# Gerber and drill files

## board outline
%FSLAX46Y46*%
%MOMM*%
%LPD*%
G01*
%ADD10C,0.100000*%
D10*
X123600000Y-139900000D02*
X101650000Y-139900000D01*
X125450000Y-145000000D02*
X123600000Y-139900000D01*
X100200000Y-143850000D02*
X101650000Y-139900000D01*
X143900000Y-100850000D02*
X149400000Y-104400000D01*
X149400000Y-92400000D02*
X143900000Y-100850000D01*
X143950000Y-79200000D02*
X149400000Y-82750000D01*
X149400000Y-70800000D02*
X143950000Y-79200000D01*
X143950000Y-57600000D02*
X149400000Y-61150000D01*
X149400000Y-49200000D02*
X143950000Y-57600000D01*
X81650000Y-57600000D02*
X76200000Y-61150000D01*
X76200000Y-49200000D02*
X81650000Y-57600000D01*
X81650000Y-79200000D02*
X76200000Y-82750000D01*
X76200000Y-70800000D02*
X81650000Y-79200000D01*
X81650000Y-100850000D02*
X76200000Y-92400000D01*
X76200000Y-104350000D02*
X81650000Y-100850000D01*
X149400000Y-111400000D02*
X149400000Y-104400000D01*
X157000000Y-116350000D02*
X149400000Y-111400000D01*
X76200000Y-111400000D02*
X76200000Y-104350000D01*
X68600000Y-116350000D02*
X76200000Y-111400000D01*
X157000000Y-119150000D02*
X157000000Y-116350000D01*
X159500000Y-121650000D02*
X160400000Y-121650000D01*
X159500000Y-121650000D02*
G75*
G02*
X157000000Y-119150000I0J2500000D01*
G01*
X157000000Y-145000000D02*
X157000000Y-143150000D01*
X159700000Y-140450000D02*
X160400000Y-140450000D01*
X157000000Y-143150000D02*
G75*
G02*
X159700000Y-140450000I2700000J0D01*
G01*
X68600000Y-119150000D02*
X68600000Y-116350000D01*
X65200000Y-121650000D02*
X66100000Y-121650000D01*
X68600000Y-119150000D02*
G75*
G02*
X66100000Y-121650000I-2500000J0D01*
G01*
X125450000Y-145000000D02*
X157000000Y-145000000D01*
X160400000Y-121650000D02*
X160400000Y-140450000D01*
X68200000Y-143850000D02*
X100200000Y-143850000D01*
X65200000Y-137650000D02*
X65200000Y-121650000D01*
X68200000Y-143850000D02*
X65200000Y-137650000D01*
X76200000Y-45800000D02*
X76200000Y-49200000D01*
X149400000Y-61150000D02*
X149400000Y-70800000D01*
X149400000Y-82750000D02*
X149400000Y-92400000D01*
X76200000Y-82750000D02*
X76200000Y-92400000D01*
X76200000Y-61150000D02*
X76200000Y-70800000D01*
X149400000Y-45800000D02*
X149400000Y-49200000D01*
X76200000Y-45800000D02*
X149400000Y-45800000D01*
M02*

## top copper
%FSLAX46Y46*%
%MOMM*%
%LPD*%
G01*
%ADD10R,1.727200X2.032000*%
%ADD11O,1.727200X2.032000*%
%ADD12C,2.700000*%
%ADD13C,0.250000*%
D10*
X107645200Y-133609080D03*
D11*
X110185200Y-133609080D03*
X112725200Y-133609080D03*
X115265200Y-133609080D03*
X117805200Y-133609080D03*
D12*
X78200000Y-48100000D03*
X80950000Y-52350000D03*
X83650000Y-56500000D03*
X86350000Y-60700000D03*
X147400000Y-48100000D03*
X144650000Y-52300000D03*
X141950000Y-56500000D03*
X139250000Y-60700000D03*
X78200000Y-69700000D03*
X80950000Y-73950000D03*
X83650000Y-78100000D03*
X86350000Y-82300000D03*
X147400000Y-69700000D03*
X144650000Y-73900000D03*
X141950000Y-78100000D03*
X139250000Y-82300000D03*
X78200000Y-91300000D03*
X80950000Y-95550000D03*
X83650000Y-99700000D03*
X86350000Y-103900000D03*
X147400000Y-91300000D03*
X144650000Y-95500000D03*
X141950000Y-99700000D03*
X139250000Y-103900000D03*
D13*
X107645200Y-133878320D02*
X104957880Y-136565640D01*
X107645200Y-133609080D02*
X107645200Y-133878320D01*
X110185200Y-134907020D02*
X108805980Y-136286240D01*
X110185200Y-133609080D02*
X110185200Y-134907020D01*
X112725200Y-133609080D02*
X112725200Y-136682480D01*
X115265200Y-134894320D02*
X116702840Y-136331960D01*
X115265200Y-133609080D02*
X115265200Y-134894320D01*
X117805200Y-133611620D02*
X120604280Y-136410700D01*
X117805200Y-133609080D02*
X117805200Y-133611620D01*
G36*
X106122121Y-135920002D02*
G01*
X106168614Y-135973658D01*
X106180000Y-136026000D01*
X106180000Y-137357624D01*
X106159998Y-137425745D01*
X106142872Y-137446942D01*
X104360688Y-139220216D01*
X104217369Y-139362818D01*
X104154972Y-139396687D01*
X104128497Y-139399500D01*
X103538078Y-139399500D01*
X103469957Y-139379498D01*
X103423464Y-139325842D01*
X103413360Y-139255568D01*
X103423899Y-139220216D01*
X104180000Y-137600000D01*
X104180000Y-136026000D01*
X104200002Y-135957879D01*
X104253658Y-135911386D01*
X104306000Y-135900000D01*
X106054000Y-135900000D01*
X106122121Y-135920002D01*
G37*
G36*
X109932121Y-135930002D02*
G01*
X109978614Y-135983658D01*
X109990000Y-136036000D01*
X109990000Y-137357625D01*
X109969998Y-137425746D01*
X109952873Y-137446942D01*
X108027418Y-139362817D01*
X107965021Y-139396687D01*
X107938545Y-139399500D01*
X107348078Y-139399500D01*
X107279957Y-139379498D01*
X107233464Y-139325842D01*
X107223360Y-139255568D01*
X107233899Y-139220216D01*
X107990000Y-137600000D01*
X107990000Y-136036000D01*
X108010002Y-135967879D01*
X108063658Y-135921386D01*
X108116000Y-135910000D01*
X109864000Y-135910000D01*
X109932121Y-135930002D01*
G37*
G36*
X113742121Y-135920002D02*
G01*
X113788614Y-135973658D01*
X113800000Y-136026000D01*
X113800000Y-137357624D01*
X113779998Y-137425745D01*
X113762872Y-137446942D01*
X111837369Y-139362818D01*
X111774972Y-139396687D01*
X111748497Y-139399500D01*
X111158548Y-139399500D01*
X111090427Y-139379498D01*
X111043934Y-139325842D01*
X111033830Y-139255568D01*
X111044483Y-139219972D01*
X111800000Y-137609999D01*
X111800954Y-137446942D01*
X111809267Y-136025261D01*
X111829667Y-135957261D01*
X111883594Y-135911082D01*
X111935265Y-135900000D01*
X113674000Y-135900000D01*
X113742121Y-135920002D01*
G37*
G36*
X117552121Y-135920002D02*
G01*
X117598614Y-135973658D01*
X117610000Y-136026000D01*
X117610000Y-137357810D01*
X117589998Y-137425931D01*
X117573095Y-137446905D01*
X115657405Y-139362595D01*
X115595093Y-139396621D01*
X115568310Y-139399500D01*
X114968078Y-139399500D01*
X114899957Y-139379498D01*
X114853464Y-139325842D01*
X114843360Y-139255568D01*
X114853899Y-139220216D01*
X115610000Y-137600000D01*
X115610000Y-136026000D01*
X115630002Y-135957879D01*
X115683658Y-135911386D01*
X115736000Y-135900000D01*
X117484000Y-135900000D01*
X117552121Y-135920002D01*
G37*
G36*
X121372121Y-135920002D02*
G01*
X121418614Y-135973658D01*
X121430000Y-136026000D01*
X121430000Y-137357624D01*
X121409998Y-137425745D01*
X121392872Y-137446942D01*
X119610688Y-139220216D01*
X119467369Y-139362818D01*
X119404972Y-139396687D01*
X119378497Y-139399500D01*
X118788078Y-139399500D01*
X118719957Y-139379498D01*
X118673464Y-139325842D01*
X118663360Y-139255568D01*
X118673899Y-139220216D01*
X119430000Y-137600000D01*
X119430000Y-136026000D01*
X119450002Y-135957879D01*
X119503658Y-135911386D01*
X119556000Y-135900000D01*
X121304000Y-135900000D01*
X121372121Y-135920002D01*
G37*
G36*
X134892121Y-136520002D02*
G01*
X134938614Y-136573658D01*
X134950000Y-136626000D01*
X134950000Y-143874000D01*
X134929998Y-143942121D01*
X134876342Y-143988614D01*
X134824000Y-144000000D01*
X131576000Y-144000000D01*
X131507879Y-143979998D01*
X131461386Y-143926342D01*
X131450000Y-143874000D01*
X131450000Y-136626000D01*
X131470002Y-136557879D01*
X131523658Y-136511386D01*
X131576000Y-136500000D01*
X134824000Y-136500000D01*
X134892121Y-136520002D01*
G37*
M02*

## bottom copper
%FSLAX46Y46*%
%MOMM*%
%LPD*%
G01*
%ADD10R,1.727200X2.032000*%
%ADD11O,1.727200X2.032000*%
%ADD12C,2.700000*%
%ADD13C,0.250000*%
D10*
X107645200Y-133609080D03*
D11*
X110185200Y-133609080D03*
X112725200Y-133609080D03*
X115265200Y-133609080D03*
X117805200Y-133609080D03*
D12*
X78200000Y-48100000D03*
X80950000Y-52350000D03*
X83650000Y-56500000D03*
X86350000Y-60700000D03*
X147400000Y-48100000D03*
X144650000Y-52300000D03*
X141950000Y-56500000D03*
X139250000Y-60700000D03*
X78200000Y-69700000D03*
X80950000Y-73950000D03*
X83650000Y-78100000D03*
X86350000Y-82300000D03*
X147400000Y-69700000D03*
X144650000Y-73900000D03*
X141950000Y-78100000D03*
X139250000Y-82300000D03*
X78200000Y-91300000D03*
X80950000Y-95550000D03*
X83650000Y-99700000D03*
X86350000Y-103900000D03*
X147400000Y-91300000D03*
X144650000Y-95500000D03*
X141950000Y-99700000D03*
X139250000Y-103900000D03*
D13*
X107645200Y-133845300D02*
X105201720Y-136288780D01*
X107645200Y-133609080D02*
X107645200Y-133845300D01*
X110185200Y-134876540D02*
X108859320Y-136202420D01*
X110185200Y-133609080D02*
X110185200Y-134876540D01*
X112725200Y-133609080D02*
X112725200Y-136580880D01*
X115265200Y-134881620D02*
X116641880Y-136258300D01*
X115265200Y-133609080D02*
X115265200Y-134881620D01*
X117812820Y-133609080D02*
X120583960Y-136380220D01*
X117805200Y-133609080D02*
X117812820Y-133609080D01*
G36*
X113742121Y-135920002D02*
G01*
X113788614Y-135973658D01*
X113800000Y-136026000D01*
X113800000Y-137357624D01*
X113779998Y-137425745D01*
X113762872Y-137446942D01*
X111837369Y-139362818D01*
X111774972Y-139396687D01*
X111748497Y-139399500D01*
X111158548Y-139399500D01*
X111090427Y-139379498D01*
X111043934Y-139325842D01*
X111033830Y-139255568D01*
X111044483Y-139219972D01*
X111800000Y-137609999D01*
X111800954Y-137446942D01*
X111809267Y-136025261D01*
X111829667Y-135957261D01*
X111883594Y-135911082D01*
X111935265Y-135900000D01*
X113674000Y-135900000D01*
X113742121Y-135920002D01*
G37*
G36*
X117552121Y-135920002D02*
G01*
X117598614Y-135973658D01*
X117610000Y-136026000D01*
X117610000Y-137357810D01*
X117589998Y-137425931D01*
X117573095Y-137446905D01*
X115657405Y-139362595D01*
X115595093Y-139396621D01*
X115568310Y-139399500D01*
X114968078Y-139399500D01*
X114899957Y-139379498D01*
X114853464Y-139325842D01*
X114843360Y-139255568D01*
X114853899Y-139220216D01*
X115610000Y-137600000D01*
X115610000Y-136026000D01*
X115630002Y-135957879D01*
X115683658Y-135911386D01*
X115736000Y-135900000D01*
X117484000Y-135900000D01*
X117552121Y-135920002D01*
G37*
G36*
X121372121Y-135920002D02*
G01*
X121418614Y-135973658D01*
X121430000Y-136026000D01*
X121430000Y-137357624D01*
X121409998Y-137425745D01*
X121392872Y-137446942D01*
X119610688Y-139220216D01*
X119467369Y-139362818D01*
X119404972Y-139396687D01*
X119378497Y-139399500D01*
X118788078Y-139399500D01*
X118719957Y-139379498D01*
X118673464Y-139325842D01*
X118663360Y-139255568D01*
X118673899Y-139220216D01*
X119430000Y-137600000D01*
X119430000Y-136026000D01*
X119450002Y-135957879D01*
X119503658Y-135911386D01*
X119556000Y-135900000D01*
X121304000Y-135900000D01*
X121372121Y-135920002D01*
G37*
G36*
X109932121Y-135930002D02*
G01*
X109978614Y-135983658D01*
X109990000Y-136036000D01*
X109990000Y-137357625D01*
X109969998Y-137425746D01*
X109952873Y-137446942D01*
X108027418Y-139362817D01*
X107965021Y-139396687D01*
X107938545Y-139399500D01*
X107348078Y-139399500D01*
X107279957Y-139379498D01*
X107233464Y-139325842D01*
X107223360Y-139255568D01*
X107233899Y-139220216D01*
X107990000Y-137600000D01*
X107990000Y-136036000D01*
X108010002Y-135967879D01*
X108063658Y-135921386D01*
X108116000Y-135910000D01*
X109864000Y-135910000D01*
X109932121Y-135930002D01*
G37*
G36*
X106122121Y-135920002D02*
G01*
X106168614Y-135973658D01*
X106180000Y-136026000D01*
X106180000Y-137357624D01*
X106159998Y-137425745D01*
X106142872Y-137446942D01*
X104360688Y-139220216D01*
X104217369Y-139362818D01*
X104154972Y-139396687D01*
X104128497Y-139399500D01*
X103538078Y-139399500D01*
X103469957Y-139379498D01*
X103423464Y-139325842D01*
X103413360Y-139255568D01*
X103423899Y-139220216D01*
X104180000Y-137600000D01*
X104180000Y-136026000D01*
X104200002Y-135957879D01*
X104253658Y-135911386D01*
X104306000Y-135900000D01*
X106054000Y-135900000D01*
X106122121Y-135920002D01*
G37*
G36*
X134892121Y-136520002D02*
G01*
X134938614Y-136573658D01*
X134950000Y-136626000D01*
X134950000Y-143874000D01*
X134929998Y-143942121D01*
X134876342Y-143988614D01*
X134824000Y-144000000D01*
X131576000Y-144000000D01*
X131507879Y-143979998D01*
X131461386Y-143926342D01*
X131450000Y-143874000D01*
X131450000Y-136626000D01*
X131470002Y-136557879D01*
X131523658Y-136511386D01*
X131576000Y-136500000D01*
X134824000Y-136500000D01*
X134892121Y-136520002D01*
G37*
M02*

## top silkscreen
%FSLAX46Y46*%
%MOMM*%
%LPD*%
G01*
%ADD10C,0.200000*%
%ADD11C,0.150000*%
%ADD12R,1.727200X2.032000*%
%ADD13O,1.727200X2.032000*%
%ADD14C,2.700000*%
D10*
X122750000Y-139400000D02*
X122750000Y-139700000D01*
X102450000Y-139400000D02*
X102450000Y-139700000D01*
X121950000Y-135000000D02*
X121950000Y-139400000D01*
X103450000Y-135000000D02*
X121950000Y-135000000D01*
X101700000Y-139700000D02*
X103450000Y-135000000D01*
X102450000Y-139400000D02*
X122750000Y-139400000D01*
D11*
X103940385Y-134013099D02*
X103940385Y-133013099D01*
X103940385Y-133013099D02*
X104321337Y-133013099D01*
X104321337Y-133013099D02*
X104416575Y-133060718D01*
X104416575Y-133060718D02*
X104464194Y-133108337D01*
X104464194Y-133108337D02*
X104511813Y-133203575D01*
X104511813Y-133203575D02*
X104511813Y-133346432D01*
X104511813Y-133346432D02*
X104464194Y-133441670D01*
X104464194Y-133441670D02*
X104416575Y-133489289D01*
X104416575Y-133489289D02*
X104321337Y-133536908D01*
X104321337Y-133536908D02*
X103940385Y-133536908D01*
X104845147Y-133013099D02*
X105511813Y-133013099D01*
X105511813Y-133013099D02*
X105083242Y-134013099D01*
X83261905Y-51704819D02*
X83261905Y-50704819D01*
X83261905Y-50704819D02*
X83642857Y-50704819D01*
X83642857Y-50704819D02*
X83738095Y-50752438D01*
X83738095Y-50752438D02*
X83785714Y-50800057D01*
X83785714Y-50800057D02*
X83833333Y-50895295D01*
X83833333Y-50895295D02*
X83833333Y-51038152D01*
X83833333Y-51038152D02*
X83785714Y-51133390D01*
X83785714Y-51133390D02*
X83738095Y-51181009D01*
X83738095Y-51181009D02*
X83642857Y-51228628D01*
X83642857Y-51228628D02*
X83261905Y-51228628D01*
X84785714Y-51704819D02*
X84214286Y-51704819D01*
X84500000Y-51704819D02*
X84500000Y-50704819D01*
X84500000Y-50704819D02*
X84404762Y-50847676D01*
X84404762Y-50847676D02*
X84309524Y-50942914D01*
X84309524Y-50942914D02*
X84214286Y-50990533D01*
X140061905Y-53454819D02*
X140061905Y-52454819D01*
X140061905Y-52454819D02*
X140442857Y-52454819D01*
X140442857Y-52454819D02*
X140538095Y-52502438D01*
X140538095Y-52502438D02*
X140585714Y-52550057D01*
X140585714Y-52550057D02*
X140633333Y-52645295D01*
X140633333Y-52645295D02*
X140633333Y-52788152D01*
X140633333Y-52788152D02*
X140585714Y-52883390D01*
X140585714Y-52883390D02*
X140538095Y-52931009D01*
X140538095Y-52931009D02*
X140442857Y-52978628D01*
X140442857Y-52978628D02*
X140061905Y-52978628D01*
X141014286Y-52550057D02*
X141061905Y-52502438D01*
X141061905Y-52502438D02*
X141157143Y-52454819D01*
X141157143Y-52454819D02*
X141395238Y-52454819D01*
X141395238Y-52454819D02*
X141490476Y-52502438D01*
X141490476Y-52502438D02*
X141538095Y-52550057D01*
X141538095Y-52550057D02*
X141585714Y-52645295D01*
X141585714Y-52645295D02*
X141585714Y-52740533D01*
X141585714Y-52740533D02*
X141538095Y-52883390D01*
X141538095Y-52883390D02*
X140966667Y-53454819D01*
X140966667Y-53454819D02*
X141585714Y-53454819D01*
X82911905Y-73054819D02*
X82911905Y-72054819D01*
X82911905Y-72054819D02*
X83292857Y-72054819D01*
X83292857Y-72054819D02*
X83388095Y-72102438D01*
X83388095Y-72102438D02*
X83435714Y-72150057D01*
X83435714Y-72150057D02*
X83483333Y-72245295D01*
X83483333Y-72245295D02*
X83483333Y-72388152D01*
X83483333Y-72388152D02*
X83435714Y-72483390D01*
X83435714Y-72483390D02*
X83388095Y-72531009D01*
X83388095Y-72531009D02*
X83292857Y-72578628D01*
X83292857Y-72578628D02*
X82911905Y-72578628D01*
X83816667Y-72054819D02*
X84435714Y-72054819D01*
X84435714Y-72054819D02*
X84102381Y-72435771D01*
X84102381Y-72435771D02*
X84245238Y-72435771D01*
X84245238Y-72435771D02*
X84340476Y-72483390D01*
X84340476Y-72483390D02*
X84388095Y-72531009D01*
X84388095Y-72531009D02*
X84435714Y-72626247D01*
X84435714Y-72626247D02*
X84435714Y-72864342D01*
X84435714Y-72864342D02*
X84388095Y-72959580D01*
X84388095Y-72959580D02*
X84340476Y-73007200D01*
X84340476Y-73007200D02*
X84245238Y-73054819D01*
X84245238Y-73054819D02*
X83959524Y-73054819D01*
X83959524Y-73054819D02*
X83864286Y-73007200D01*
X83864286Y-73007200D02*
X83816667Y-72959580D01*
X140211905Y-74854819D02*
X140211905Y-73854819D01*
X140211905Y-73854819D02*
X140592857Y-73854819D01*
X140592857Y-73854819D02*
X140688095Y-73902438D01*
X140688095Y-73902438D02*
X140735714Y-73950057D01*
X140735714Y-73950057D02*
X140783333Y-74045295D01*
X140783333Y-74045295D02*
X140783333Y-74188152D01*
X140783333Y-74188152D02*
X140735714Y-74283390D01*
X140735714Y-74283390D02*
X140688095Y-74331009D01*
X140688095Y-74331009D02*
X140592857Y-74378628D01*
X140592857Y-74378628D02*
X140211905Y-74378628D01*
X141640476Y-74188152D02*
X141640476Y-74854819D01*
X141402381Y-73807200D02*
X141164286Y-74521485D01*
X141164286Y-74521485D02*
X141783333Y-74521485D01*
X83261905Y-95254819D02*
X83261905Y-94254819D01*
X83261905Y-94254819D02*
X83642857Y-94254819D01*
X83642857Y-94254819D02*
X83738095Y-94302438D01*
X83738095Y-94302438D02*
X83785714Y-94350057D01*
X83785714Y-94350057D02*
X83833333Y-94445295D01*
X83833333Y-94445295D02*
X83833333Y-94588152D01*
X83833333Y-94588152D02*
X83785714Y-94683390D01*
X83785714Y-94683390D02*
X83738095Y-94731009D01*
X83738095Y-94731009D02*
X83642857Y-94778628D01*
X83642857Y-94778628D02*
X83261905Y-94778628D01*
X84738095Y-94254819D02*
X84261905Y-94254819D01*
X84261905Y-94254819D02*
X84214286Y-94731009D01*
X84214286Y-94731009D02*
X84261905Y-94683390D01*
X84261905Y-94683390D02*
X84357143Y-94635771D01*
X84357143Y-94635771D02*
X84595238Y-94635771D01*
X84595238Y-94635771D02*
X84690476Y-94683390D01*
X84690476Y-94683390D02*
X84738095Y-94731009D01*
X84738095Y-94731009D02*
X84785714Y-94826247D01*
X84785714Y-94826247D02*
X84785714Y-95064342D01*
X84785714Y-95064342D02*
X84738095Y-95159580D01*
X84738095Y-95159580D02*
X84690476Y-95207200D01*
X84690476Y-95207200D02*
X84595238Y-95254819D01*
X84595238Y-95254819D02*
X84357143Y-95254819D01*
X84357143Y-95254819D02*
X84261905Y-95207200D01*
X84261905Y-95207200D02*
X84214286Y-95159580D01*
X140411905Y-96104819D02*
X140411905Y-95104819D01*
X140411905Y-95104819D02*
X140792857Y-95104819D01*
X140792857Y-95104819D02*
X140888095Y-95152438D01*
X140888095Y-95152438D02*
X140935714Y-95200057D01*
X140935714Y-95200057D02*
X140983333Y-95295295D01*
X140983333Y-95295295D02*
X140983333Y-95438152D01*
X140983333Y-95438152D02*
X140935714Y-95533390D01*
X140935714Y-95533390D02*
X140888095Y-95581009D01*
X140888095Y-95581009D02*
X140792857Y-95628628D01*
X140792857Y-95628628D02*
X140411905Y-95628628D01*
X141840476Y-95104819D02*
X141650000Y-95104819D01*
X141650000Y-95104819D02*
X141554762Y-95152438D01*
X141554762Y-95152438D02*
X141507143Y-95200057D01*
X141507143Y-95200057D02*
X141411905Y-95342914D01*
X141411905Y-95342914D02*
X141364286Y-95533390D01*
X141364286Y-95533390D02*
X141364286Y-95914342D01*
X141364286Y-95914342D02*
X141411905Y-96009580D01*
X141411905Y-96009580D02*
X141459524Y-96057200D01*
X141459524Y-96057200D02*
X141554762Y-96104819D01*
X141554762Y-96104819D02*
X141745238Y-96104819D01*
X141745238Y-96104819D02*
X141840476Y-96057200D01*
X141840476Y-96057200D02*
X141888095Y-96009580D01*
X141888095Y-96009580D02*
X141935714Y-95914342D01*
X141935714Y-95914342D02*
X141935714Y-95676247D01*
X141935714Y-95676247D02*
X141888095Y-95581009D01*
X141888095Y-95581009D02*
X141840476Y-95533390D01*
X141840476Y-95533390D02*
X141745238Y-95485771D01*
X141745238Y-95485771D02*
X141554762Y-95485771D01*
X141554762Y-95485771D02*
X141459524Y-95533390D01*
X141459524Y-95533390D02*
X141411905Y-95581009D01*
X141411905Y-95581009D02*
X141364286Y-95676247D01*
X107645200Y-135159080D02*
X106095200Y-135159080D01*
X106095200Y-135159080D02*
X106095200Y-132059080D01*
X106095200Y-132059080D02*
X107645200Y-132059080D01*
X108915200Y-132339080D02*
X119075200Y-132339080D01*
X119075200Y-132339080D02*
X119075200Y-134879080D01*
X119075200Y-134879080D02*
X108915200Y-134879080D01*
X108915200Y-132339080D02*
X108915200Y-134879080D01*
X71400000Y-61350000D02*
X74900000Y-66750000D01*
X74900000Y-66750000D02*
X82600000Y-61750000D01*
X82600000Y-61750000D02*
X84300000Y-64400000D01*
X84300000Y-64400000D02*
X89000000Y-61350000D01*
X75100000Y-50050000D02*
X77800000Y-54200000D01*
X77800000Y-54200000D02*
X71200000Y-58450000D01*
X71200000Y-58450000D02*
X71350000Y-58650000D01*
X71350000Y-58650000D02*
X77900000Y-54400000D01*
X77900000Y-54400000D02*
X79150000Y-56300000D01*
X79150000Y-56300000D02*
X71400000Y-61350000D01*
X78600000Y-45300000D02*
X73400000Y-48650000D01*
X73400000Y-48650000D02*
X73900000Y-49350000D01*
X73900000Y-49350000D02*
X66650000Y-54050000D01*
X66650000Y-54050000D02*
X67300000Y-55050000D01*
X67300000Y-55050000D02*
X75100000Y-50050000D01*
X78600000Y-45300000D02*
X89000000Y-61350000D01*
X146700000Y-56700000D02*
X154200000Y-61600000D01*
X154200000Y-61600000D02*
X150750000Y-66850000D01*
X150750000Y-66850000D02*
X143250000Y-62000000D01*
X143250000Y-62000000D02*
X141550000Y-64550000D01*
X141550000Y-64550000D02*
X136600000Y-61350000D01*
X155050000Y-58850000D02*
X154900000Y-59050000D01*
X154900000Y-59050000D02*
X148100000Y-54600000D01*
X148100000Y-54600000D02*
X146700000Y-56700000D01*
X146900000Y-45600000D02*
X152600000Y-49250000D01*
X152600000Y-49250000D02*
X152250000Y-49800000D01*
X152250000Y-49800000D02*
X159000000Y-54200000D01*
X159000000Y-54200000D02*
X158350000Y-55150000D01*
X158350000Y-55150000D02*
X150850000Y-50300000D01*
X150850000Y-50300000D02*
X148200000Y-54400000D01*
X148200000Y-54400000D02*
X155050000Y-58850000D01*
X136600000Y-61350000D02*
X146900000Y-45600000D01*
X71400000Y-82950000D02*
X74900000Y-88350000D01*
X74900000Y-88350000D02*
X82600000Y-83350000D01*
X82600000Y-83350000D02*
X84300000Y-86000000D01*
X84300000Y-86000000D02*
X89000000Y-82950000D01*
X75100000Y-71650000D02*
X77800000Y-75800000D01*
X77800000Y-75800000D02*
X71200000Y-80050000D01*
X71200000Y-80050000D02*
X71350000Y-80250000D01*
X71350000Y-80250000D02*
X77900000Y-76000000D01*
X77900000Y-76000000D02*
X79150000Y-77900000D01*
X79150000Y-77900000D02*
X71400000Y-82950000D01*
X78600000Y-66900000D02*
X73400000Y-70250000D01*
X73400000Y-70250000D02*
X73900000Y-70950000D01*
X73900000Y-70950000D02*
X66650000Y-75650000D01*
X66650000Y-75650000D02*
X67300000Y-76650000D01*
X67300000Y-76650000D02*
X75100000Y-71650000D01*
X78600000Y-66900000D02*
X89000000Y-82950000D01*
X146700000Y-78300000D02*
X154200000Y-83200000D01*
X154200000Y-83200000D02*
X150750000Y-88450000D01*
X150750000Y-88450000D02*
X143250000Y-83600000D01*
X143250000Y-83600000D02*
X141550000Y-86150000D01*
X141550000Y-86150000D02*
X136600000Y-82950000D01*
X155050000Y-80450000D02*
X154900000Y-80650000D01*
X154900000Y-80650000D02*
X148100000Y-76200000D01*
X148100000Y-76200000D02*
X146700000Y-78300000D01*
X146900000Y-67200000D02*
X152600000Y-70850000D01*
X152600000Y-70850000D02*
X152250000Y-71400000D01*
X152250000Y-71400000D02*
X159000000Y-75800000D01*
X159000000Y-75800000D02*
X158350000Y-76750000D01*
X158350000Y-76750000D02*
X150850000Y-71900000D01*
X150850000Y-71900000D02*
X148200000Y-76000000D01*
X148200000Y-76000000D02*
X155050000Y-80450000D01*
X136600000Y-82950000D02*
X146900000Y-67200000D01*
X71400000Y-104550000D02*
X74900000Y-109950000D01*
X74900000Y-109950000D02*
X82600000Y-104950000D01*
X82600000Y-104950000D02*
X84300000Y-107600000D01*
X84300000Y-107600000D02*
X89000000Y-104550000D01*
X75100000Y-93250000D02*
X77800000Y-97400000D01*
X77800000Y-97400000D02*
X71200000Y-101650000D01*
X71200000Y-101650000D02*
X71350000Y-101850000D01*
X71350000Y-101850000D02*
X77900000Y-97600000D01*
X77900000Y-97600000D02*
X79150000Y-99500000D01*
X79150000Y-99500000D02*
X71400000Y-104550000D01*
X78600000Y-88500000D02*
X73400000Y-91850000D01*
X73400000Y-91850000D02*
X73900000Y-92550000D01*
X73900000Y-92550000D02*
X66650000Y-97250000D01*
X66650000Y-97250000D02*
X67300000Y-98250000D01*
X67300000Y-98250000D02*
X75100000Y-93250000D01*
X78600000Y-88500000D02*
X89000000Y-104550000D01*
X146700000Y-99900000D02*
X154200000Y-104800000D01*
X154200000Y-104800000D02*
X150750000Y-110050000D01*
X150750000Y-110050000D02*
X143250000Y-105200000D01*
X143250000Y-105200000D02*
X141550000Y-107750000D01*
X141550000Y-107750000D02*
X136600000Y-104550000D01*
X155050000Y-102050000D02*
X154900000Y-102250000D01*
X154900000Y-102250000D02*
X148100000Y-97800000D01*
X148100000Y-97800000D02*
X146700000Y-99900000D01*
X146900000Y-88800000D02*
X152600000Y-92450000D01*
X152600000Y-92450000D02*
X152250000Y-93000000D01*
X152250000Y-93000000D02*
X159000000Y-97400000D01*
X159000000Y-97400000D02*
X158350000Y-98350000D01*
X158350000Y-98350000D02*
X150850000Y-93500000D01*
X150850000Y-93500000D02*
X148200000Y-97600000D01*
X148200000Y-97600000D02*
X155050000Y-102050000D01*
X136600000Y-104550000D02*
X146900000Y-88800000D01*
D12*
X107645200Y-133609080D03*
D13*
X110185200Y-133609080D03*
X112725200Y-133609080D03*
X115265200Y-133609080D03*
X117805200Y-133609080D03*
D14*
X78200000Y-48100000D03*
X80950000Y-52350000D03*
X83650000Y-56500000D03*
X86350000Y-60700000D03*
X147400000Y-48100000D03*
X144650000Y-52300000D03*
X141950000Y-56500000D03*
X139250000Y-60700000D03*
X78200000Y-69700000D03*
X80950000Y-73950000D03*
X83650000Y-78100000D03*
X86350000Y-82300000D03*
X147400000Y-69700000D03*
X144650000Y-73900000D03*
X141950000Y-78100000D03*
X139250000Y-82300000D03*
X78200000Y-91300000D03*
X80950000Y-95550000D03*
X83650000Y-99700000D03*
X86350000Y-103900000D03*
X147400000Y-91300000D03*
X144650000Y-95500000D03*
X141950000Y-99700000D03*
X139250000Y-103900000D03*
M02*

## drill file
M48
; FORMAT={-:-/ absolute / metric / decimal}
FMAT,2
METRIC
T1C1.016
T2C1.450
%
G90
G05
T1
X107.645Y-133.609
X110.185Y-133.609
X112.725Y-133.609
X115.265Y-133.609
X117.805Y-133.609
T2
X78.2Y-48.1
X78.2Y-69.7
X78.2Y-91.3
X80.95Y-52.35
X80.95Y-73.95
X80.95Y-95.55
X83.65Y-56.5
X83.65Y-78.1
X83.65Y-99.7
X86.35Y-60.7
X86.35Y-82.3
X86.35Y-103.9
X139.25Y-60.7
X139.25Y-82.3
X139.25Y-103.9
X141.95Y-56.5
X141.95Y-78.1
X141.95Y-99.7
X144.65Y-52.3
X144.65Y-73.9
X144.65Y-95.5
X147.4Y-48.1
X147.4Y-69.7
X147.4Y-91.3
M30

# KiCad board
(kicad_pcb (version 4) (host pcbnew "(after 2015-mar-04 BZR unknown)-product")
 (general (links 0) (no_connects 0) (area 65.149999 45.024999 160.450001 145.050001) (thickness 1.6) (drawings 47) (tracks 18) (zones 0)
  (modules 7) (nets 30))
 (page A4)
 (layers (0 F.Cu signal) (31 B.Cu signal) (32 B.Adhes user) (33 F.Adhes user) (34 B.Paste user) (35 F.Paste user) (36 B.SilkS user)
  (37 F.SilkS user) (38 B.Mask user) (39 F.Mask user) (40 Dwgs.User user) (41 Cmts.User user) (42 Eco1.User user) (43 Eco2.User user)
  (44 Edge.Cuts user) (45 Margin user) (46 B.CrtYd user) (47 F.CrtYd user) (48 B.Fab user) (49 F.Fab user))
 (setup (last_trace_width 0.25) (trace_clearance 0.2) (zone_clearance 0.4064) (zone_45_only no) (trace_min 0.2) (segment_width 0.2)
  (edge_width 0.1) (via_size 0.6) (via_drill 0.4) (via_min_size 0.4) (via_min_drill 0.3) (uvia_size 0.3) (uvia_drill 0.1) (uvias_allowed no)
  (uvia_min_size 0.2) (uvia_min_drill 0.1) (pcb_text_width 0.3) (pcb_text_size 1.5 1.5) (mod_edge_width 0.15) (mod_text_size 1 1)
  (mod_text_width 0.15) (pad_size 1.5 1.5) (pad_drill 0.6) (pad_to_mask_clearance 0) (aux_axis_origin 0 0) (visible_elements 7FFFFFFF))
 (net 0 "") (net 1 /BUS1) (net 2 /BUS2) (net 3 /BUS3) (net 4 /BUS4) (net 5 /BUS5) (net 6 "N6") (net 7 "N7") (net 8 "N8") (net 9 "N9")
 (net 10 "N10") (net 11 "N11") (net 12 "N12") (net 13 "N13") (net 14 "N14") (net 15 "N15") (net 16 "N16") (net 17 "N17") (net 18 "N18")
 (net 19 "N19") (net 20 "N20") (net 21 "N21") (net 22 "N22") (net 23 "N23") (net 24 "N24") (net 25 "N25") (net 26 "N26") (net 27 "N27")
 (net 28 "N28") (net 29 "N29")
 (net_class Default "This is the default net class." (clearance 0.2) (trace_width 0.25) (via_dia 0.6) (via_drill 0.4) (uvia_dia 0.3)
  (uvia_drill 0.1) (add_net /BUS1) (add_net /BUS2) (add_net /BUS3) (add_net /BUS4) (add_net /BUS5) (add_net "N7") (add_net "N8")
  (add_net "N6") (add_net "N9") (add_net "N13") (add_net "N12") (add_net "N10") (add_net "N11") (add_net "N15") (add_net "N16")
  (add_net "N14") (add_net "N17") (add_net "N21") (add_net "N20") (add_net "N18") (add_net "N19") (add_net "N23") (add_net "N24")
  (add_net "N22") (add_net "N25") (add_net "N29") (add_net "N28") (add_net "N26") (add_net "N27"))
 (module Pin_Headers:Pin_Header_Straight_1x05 (layer F.Cu) (at 107.6452 133.60908 90)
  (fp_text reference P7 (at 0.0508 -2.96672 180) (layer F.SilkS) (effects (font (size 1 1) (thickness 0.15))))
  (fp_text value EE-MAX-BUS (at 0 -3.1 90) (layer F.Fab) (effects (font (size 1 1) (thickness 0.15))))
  (fp_line (start -1.55 0) (end -1.55 -1.55) (layer F.SilkS) (width 0.15))
  (fp_line (start -1.55 -1.55) (end 1.55 -1.55) (layer F.SilkS) (width 0.15))
  (fp_line (start 1.55 -1.55) (end 1.55 0) (layer F.SilkS) (width 0.15))
  (fp_line (start 1.27 1.27) (end 1.27 11.43) (layer F.SilkS) (width 0.15))
  (fp_line (start 1.27 11.43) (end -1.27 11.43) (layer F.SilkS) (width 0.15))
  (fp_line (start -1.27 11.43) (end -1.27 1.27) (layer F.SilkS) (width 0.15))
  (fp_line (start 1.27 1.27) (end -1.27 1.27) (layer F.SilkS) (width 0.15))
  (pad 1 thru_hole rect (at 0 0 90) (size 2.032 1.7272) (drill 1.016) (layers *.Cu *.Mask F.SilkS) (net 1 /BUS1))
  (pad 2 thru_hole oval (at 0 2.54 90) (size 2.032 1.7272) (drill 1.016) (layers *.Cu *.Mask F.SilkS) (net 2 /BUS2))
  (pad 3 thru_hole oval (at 0 5.08 90) (size 2.032 1.7272) (drill 1.016) (layers *.Cu *.Mask F.SilkS) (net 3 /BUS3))
  (pad 4 thru_hole oval (at 0 7.62 90) (size 2.032 1.7272) (drill 1.016) (layers *.Cu *.Mask F.SilkS) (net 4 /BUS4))
  (pad 5 thru_hole oval (at 0 10.16 90) (size 2.032 1.7272) (drill 1.016) (layers *.Cu *.Mask F.SilkS) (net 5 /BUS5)))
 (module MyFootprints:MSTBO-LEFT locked (layer F.Cu) (at 78.2 48.1)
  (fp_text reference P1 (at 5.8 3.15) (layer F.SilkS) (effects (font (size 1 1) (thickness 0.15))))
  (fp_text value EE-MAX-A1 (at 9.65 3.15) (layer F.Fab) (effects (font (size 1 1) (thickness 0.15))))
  (fp_line (start -6.8 13.25) (end -3.3 18.65) (layer F.SilkS) (width 0.15))
  (fp_line (start -3.3 18.65) (end 4.4 13.65) (layer F.SilkS) (width 0.15))
  (fp_line (start 4.4 13.65) (end 6.1 16.3) (layer F.SilkS) (width 0.15))
  (fp_line (start 6.1 16.3) (end 10.8 13.25) (layer F.SilkS) (width 0.15))
  (fp_line (start -3.1 1.95) (end -0.4 6.1) (layer F.SilkS) (width 0.15))
  (fp_line (start -0.4 6.1) (end -7 10.35) (layer F.SilkS) (width 0.15))
  (fp_line (start -7 10.35) (end -6.85 10.55) (layer F.SilkS) (width 0.15))
  (fp_line (start -6.85 10.55) (end -0.3 6.3) (layer F.SilkS) (width 0.15))
  (fp_line (start -0.3 6.3) (end 0.95 8.2) (layer F.SilkS) (width 0.15))
  (fp_line (start 0.95 8.2) (end -6.8 13.25) (layer F.SilkS) (width 0.15))
  (fp_line (start 0.4 -2.8) (end -4.8 0.55) (layer F.SilkS) (width 0.15))
  (fp_line (start -4.8 0.55) (end -4.3 1.25) (layer F.SilkS) (width 0.15))
  (fp_line (start -4.3 1.25) (end -11.55 5.95) (layer F.SilkS) (width 0.15))
  (fp_line (start -11.55 5.95) (end -10.9 6.95) (layer F.SilkS) (width 0.15))
  (fp_line (start -10.9 6.95) (end -3.1 1.95) (layer F.SilkS) (width 0.15))
  (fp_line (start 0.4 -2.8) (end 10.8 13.25) (layer F.SilkS) (width 0.15))
  (pad 3 thru_hole circle (at 0 0) (size 2.7 2.7) (drill 1.45) (layers *.Cu *.Mask F.SilkS) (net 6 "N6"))
  (pad 1 thru_hole circle (at 2.75 4.25) (size 2.7 2.7) (drill 1.45) (layers *.Cu *.Mask F.SilkS) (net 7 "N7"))
  (pad 2 thru_hole circle (at 5.45 8.4) (size 2.7 2.7) (drill 1.45) (layers *.Cu *.Mask F.SilkS) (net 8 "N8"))
  (pad 4 thru_hole circle (at 8.15 12.6) (size 2.7 2.7) (drill 1.45) (layers *.Cu *.Mask F.SilkS) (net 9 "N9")))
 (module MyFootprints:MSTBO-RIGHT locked (layer F.Cu) (at 147.4 48.1)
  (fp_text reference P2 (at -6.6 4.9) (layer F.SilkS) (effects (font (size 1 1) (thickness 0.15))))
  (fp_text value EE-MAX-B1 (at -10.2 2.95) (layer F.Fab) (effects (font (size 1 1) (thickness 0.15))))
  (fp_line (start -0.7 8.6) (end 6.8 13.5) (layer F.SilkS) (width 0.15))
  (fp_line (start 6.8 13.5) (end 3.35 18.75) (layer F.SilkS) (width 0.15))
  (fp_line (start 3.35 18.75) (end -4.15 13.9) (layer F.SilkS) (width 0.15))
  (fp_line (start -4.15 13.9) (end -5.85 16.45) (layer F.SilkS) (width 0.15))
  (fp_line (start -5.85 16.45) (end -10.8 13.25) (layer F.SilkS) (width 0.15))
  (fp_line (start 7.65 10.75) (end 7.5 10.95) (layer F.SilkS) (width 0.15))
  (fp_line (start 7.5 10.95) (end 0.7 6.5) (layer F.SilkS) (width 0.15))
  (fp_line (start 0.7 6.5) (end -0.7 8.6) (layer F.SilkS) (width 0.15))
  (fp_line (start -0.5 -2.5) (end 5.2 1.15) (layer F.SilkS) (width 0.15))
  (fp_line (start 5.2 1.15) (end 4.85 1.7) (layer F.SilkS) (width 0.15))
  (fp_line (start 4.85 1.7) (end 11.6 6.1) (layer F.SilkS) (width 0.15))
  (fp_line (start 11.6 6.1) (end 10.95 7.05) (layer F.SilkS) (width 0.15))
  (fp_line (start 10.95 7.05) (end 3.45 2.2) (layer F.SilkS) (width 0.15))
  (fp_line (start 3.45 2.2) (end 0.8 6.3) (layer F.SilkS) (width 0.15))
  (fp_line (start 0.8 6.3) (end 7.65 10.75) (layer F.SilkS) (width 0.15))
  (fp_line (start -10.8 13.25) (end -0.5 -2.5) (layer F.SilkS) (width 0.15))
  (pad 3 thru_hole circle (at 0 0) (size 2.7 2.7) (drill 1.45) (layers *.Cu *.Mask F.SilkS) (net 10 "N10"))
  (pad 4 thru_hole circle (at -2.75 4.2) (size 2.7 2.7) (drill 1.45) (layers *.Cu *.Mask F.SilkS) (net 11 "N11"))
  (pad 2 thru_hole circle (at -5.45 8.4) (size 2.7 2.7) (drill 1.45) (layers *.Cu *.Mask F.SilkS) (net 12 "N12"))
  (pad 1 thru_hole circle (at -8.15 12.6) (size 2.7 2.7) (drill 1.45) (layers *.Cu *.Mask F.SilkS) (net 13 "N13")))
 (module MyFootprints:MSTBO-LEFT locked (layer F.Cu) (at 78.2 69.7)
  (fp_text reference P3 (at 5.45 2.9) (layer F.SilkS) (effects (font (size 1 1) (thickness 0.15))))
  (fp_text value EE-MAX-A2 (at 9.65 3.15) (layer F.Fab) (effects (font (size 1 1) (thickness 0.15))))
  (fp_line (start -6.8 13.25) (end -3.3 18.65) (layer F.SilkS) (width 0.15))
  (fp_line (start -3.3 18.65) (end 4.4 13.65) (layer F.SilkS) (width 0.15))
  (fp_line (start 4.4 13.65) (end 6.1 16.3) (layer F.SilkS) (width 0.15))
  (fp_line (start 6.1 16.3) (end 10.8 13.25) (layer F.SilkS) (width 0.15))
  (fp_line (start -3.1 1.95) (end -0.4 6.1) (layer F.SilkS) (width 0.15))
  (fp_line (start -0.4 6.1) (end -7 10.35) (layer F.SilkS) (width 0.15))
  (fp_line (start -7 10.35) (end -6.85 10.55) (layer F.SilkS) (width 0.15))
  (fp_line (start -6.85 10.55) (end -0.3 6.3) (layer F.SilkS) (width 0.15))
  (fp_line (start -0.3 6.3) (end 0.95 8.2) (layer F.SilkS) (width 0.15))
  (fp_line (start 0.95 8.2) (end -6.8 13.25) (layer F.SilkS) (width 0.15))
  (fp_line (start 0.4 -2.8) (end -4.8 0.55) (layer F.SilkS) (width 0.15))
  (fp_line (start -4.8 0.55) (end -4.3 1.25) (layer F.SilkS) (width 0.15))
  (fp_line (start -4.3 1.25) (end -11.55 5.95) (layer F.SilkS) (width 0.15))
  (fp_line (start -11.55 5.95) (end -10.9 6.95) (layer F.SilkS) (width 0.15))
  (fp_line (start -10.9 6.95) (end -3.1 1.95) (layer F.SilkS) (width 0.15))
  (fp_line (start 0.4 -2.8) (end 10.8 13.25) (layer F.SilkS) (width 0.15))
  (pad 3 thru_hole circle (at 0 0) (size 2.7 2.7) (drill 1.45) (layers *.Cu *.Mask F.SilkS) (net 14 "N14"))
  (pad 1 thru_hole circle (at 2.75 4.25) (size 2.7 2.7) (drill 1.45) (layers *.Cu *.Mask F.SilkS) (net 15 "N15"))
  (pad 2 thru_hole circle (at 5.45 8.4) (size 2.7 2.7) (drill 1.45) (layers *.Cu *.Mask F.SilkS) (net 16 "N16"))
  (pad 4 thru_hole circle (at 8.15 12.6) (size 2.7 2.7) (drill 1.45) (layers *.Cu *.Mask F.SilkS) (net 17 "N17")))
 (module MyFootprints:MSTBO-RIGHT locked (layer F.Cu) (at 147.4 69.7)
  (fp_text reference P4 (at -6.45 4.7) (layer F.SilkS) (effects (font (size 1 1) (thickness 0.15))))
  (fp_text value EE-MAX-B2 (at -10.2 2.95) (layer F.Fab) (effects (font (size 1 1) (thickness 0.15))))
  (fp_line (start -0.7 8.6) (end 6.8 13.5) (layer F.SilkS) (width 0.15))
  (fp_line (start 6.8 13.5) (end 3.35 18.75) (layer F.SilkS) (width 0.15))
  (fp_line (start 3.35 18.75) (end -4.15 13.9) (layer F.SilkS) (width 0.15))
  (fp_line (start -4.15 13.9) (end -5.85 16.45) (layer F.SilkS) (width 0.15))
  (fp_line (start -5.85 16.45) (end -10.8 13.25) (layer F.SilkS) (width 0.15))
  (fp_line (start 7.65 10.75) (end 7.5 10.95) (layer F.SilkS) (width 0.15))
  (fp_line (start 7.5 10.95) (end 0.7 6.5) (layer F.SilkS) (width 0.15))
  (fp_line (start 0.7 6.5) (end -0.7 8.6) (layer F.SilkS) (width 0.15))
  (fp_line (start -0.5 -2.5) (end 5.2 1.15) (layer F.SilkS) (width 0.15))
  (fp_line (start 5.2 1.15) (end 4.85 1.7) (layer F.SilkS) (width 0.15))
  (fp_line (start 4.85 1.7) (end 11.6 6.1) (layer F.SilkS) (width 0.15))
  (fp_line (start 11.6 6.1) (end 10.95 7.05) (layer F.SilkS) (width 0.15))
  (fp_line (start 10.95 7.05) (end 3.45 2.2) (layer F.SilkS) (width 0.15))
  (fp_line (start 3.45 2.2) (end 0.8 6.3) (layer F.SilkS) (width 0.15))
  (fp_line (start 0.8 6.3) (end 7.65 10.75) (layer F.SilkS) (width 0.15))
  (fp_line (start -10.8 13.25) (end -0.5 -2.5) (layer F.SilkS) (width 0.15))
  (pad 3 thru_hole circle (at 0 0) (size 2.7 2.7) (drill 1.45) (layers *.Cu *.Mask F.SilkS) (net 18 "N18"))
  (pad 4 thru_hole circle (at -2.75 4.2) (size 2.7 2.7) (drill 1.45) (layers *.Cu *.Mask F.SilkS) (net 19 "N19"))
  (pad 2 thru_hole circle (at -5.45 8.4) (size 2.7 2.7) (drill 1.45) (layers *.Cu *.Mask F.SilkS) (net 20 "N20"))
  (pad 1 thru_hole circle (at -8.15 12.6) (size 2.7 2.7) (drill 1.45) (layers *.Cu *.Mask F.SilkS) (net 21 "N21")))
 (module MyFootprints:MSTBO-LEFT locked (layer F.Cu) (at 78.2 91.3)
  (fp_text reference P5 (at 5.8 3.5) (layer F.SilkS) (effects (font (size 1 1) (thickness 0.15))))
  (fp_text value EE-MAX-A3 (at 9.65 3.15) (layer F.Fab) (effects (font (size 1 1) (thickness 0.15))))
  (fp_line (start -6.8 13.25) (end -3.3 18.65) (layer F.SilkS) (width 0.15))
  (fp_line (start -3.3 18.65) (end 4.4 13.65) (layer F.SilkS) (width 0.15))
  (fp_line (start 4.4 13.65) (end 6.1 16.3) (layer F.SilkS) (width 0.15))
  (fp_line (start 6.1 16.3) (end 10.8 13.25) (layer F.SilkS) (width 0.15))
  (fp_line (start -3.1 1.95) (end -0.4 6.1) (layer F.SilkS) (width 0.15))
  (fp_line (start -0.4 6.1) (end -7 10.35) (layer F.SilkS) (width 0.15))
  (fp_line (start -7 10.35) (end -6.85 10.55) (layer F.SilkS) (width 0.15))
  (fp_line (start -6.85 10.55) (end -0.3 6.3) (layer F.SilkS) (width 0.15))
  (fp_line (start -0.3 6.3) (end 0.95 8.2) (layer F.SilkS) (width 0.15))
  (fp_line (start 0.95 8.2) (end -6.8 13.25) (layer F.SilkS) (width 0.15))
  (fp_line (start 0.4 -2.8) (end -4.8 0.55) (layer F.SilkS) (width 0.15))
  (fp_line (start -4.8 0.55) (end -4.3 1.25) (layer F.SilkS) (width 0.15))
  (fp_line (start -4.3 1.25) (end -11.55 5.95) (layer F.SilkS) (width 0.15))
  (fp_line (start -11.55 5.95) (end -10.9 6.95) (layer F.SilkS) (width 0.15))
  (fp_line (start -10.9 6.95) (end -3.1 1.95) (layer F.SilkS) (width 0.15))
  (fp_line (start 0.4 -2.8) (end 10.8 13.25) (layer F.SilkS) (width 0.15))
  (pad 3 thru_hole circle (at 0 0) (size 2.7 2.7) (drill 1.45) (layers *.Cu *.Mask F.SilkS) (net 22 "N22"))
  (pad 1 thru_hole circle (at 2.75 4.25) (size 2.7 2.7) (drill 1.45) (layers *.Cu *.Mask F.SilkS) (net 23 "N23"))
  (pad 2 thru_hole circle (at 5.45 8.4) (size 2.7 2.7) (drill 1.45) (layers *.Cu *.Mask F.SilkS) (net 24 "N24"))
  (pad 4 thru_hole circle (at 8.15 12.6) (size 2.7 2.7) (drill 1.45) (layers *.Cu *.Mask F.SilkS) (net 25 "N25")))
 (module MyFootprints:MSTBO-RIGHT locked (layer F.Cu) (at 147.4 91.3)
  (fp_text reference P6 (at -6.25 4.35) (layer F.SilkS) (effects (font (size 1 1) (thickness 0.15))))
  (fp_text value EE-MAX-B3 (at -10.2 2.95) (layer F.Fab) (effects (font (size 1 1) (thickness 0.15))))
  (fp_line (start -0.7 8.6) (end 6.8 13.5) (layer F.SilkS) (width 0.15))
  (fp_line (start 6.8 13.5) (end 3.35 18.75) (layer F.SilkS) (width 0.15))
  (fp_line (start 3.35 18.75) (end -4.15 13.9) (layer F.SilkS) (width 0.15))
  (fp_line (start -4.15 13.9) (end -5.85 16.45) (layer F.SilkS) (width 0.15))
  (fp_line (start -5.85 16.45) (end -10.8 13.25) (layer F.SilkS) (width 0.15))
  (fp_line (start 7.65 10.75) (end 7.5 10.95) (layer F.SilkS) (width 0.15))
  (fp_line (start 7.5 10.95) (end 0.7 6.5) (layer F.SilkS) (width 0.15))
  (fp_line (start 0.7 6.5) (end -0.7 8.6) (layer F.SilkS) (width 0.15))
  (fp_line (start -0.5 -2.5) (end 5.2 1.15) (layer F.SilkS) (width 0.15))
  (fp_line (start 5.2 1.15) (end 4.85 1.7) (layer F.SilkS) (width 0.15))
  (fp_line (start 4.85 1.7) (end 11.6 6.1) (layer F.SilkS) (width 0.15))
  (fp_line (start 11.6 6.1) (end 10.95 7.05) (layer F.SilkS) (width 0.15))
  (fp_line (start 10.95 7.05) (end 3.45 2.2) (layer F.SilkS) (width 0.15))
  (fp_line (start 3.45 2.2) (end 0.8 6.3) (layer F.SilkS) (width 0.15))
  (fp_line (start 0.8 6.3) (end 7.65 10.75) (layer F.SilkS) (width 0.15))
  (fp_line (start -10.8 13.25) (end -0.5 -2.5) (layer F.SilkS) (width 0.15))
  (pad 3 thru_hole circle (at 0 0) (size 2.7 2.7) (drill 1.45) (layers *.Cu *.Mask F.SilkS) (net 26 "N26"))
  (pad 4 thru_hole circle (at -2.75 4.2) (size 2.7 2.7) (drill 1.45) (layers *.Cu *.Mask F.SilkS) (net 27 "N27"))
  (pad 2 thru_hole circle (at -5.45 8.4) (size 2.7 2.7) (drill 1.45) (layers *.Cu *.Mask F.SilkS) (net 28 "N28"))
  (pad 1 thru_hole circle (at -8.15 12.6) (size 2.7 2.7) (drill 1.45) (layers *.Cu *.Mask F.SilkS) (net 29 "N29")))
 (gr_line (start 122.75 139.4) (end 122.75 139.7) (angle 90) (layer F.SilkS) (width 0.2))
 (gr_line (start 102.45 139.4) (end 102.45 139.7) (angle 90) (layer F.SilkS) (width 0.2))
 (gr_line (start 121.95 135) (end 121.95 139.4) (angle 90) (layer F.SilkS) (width 0.2))
 (gr_line (start 103.45 135) (end 121.95 135) (angle 90) (layer F.SilkS) (width 0.2))
 (gr_line (start 101.7 139.7) (end 103.45 135) (angle 90) (layer F.SilkS) (width 0.2))
 (gr_line (start 102.45 139.4) (end 122.75 139.4) (angle 90) (layer F.SilkS) (width 0.2))
 (gr_line (start 123.6 139.9) (end 101.65 139.9) (angle 90) (layer Edge.Cuts) (width 0.1))
 (gr_line (start 125.45 145) (end 123.6 139.9) (angle 90) (layer Edge.Cuts) (width 0.1))
 (gr_line (start 100.2 143.85) (end 101.65 139.9) (angle 90) (layer Edge.Cuts) (width 0.1))
 (gr_line (start 143.9 100.85) (end 149.4 104.4) (angle 90) (layer Edge.Cuts) (width 0.1))
 (gr_line (start 149.4 92.4) (end 143.9 100.85) (angle 90) (layer Edge.Cuts) (width 0.1))
 (gr_line (start 143.95 79.2) (end 149.4 82.75) (angle 90) (layer Edge.Cuts) (width 0.1))
 (gr_line (start 149.4 70.8) (end 143.95 79.2) (angle 90) (layer Edge.Cuts) (width 0.1))
 (gr_line (start 143.95 57.6) (end 149.4 61.15) (angle 90) (layer Edge.Cuts) (width 0.1))
 (gr_line (start 149.4 49.2) (end 143.95 57.6) (angle 90) (layer Edge.Cuts) (width 0.1))
 (gr_line (start 81.65 57.6) (end 76.2 61.15) (angle 90) (layer Edge.Cuts) (width 0.1))
 (gr_line (start 76.2 49.2) (end 81.65 57.6) (angle 90) (layer Edge.Cuts) (width 0.1))
 (gr_line (start 81.65 79.2) (end 76.2 82.75) (angle 90) (layer Edge.Cuts) (width 0.1))
 (gr_line (start 76.2 70.8) (end 81.65 79.2) (angle 90) (layer Edge.Cuts) (width 0.1))
 (gr_line (start 81.65 100.85) (end 76.2 92.4) (angle 90) (layer Edge.Cuts) (width 0.1))
 (gr_line (start 76.2 104.35) (end 81.65 100.85) (angle 90) (layer Edge.Cuts) (width 0.1))
 (gr_line (start 149.4 111.4) (end 149.4 104.4) (angle 90) (layer Edge.Cuts) (width 0.1))
 (gr_line (start 157 116.35) (end 149.4 111.4) (angle 90) (layer Edge.Cuts) (width 0.1))
 (gr_line (start 76.2 111.4) (end 76.2 104.35) (angle 90) (layer Edge.Cuts) (width 0.1))
 (gr_line (start 68.6 116.35) (end 76.2 111.4) (angle 90) (layer Edge.Cuts) (width 0.1))
 (gr_line (start 157 119.15) (end 157 116.35) (angle 90) (layer Edge.Cuts) (width 0.1))
 (gr_line (start 159.5 121.65) (end 160.4 121.65) (angle 90) (layer Edge.Cuts) (width 0.1))
 (gr_arc (start 159.5 119.15) (end 159.5 121.65) (angle 90) (layer Edge.Cuts) (width 0.1))
 (gr_line (start 157 145) (end 157 143.15) (angle 90) (layer Edge.Cuts) (width 0.1))
 (gr_line (start 159.7 140.45) (end 160.4 140.45) (angle 90) (layer Edge.Cuts) (width 0.1))
 (gr_arc (start 159.7 143.15) (end 157 143.15) (angle 90) (layer Edge.Cuts) (width 0.1))
 (gr_line (start 68.6 119.15) (end 68.6 116.35) (angle 90) (layer Edge.Cuts) (width 0.1))
 (gr_line (start 65.2 121.65) (end 66.1 121.65) (angle 90) (layer Edge.Cuts) (width 0.1))
 (gr_arc (start 66.1 119.15) (end 68.6 119.15) (angle 90) (layer Edge.Cuts) (width 0.1))
 (gr_line (start 125.45 145) (end 157 145) (angle 90) (layer Edge.Cuts) (width 0.1))
 (gr_line (start 160.4 121.65) (end 160.4 140.45) (angle 90) (layer Edge.Cuts) (width 0.1))
 (gr_line (start 68.2 143.85) (end 100.2 143.85) (angle 90) (layer Edge.Cuts) (width 0.1))
 (gr_line (start 65.2 137.65) (end 65.2 121.65) (angle 90) (layer Edge.Cuts) (width 0.1))
 (gr_line (start 68.2 143.85) (end 65.2 137.65) (angle 90) (layer Edge.Cuts) (width 0.1))
 (gr_line (start 76.2 45.8) (end 76.2 49.2) (angle 90) (layer Edge.Cuts) (width 0.1))
 (gr_line (start 149.4 61.15) (end 149.4 70.8) (angle 90) (layer Edge.Cuts) (width 0.1))
 (gr_line (start 149.4 82.75) (end 149.4 92.4) (angle 90) (layer Edge.Cuts) (width 0.1))
 (gr_line (start 76.2 82.75) (end 76.2 92.4) (angle 90) (layer Edge.Cuts) (width 0.1))
 (gr_line (start 76.2 61.15) (end 76.2 70.8) (angle 90) (layer Edge.Cuts) (width 0.1))
 (gr_line (start 149.4 45.8) (end 149.4 49.2) (angle 90) (layer Edge.Cuts) (width 0.1))
 (gr_line (start 76.2 45.8) (end 149.4 45.8) (angle 90) (layer Edge.Cuts) (width 0.1))
 (segment (start 107.6452 133.87832) (end 104.95788 136.56564) (width 0.25) (layer F.Cu) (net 1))
 (segment (start 107.6452 133.60908) (end 107.6452 133.87832) (width 0.25) (layer F.Cu) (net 1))
 (segment (start 107.6452 133.8453) (end 105.20172 136.28878) (width 0.25) (layer B.Cu) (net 1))
 (segment (start 107.6452 133.60908) (end 107.6452 133.8453) (width 0.25) (layer B.Cu) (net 1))
 (segment (start 110.1852 134.87654) (end 108.85932 136.20242) (width 0.25) (layer B.Cu) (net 2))
 (segment (start 110.1852 133.60908) (end 110.1852 134.87654) (width 0.25) (layer B.Cu) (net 2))
 (segment (start 110.1852 134.90702) (end 108.80598 136.28624) (width 0.25) (layer F.Cu) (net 2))
 (segment (start 110.1852 133.60908) (end 110.1852 134.90702) (width 0.25) (layer F.Cu) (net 2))
 (segment (start 112.7252 133.60908) (end 112.7252 136.58088) (width 0.25) (layer B.Cu) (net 3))
 (segment (start 112.7252 133.60908) (end 112.7252 136.68248) (width 0.25) (layer F.Cu) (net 3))
 (segment (start 115.2652 134.89432) (end 116.70284 136.33196) (width 0.25) (layer F.Cu) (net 4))
 (segment (start 115.2652 133.60908) (end 115.2652 134.89432) (width 0.25) (layer F.Cu) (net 4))
 (segment (start 115.2652 134.88162) (end 116.64188 136.2583) (width 0.25) (layer B.Cu) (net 4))
 (segment (start 115.2652 133.60908) (end 115.2652 134.88162) (width 0.25) (layer B.Cu) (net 4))
 (segment (start 117.8052 133.61162) (end 120.60428 136.4107) (width 0.25) (layer F.Cu) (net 5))
 (segment (start 117.8052 133.60908) (end 117.8052 133.61162) (width 0.25) (layer F.Cu) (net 5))
 (segment (start 117.81282 133.60908) (end 120.58396 136.38022) (width 0.25) (layer B.Cu) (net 5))
 (segment (start 117.8052 133.60908) (end 117.81282 133.60908) (width 0.25) (layer B.Cu) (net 5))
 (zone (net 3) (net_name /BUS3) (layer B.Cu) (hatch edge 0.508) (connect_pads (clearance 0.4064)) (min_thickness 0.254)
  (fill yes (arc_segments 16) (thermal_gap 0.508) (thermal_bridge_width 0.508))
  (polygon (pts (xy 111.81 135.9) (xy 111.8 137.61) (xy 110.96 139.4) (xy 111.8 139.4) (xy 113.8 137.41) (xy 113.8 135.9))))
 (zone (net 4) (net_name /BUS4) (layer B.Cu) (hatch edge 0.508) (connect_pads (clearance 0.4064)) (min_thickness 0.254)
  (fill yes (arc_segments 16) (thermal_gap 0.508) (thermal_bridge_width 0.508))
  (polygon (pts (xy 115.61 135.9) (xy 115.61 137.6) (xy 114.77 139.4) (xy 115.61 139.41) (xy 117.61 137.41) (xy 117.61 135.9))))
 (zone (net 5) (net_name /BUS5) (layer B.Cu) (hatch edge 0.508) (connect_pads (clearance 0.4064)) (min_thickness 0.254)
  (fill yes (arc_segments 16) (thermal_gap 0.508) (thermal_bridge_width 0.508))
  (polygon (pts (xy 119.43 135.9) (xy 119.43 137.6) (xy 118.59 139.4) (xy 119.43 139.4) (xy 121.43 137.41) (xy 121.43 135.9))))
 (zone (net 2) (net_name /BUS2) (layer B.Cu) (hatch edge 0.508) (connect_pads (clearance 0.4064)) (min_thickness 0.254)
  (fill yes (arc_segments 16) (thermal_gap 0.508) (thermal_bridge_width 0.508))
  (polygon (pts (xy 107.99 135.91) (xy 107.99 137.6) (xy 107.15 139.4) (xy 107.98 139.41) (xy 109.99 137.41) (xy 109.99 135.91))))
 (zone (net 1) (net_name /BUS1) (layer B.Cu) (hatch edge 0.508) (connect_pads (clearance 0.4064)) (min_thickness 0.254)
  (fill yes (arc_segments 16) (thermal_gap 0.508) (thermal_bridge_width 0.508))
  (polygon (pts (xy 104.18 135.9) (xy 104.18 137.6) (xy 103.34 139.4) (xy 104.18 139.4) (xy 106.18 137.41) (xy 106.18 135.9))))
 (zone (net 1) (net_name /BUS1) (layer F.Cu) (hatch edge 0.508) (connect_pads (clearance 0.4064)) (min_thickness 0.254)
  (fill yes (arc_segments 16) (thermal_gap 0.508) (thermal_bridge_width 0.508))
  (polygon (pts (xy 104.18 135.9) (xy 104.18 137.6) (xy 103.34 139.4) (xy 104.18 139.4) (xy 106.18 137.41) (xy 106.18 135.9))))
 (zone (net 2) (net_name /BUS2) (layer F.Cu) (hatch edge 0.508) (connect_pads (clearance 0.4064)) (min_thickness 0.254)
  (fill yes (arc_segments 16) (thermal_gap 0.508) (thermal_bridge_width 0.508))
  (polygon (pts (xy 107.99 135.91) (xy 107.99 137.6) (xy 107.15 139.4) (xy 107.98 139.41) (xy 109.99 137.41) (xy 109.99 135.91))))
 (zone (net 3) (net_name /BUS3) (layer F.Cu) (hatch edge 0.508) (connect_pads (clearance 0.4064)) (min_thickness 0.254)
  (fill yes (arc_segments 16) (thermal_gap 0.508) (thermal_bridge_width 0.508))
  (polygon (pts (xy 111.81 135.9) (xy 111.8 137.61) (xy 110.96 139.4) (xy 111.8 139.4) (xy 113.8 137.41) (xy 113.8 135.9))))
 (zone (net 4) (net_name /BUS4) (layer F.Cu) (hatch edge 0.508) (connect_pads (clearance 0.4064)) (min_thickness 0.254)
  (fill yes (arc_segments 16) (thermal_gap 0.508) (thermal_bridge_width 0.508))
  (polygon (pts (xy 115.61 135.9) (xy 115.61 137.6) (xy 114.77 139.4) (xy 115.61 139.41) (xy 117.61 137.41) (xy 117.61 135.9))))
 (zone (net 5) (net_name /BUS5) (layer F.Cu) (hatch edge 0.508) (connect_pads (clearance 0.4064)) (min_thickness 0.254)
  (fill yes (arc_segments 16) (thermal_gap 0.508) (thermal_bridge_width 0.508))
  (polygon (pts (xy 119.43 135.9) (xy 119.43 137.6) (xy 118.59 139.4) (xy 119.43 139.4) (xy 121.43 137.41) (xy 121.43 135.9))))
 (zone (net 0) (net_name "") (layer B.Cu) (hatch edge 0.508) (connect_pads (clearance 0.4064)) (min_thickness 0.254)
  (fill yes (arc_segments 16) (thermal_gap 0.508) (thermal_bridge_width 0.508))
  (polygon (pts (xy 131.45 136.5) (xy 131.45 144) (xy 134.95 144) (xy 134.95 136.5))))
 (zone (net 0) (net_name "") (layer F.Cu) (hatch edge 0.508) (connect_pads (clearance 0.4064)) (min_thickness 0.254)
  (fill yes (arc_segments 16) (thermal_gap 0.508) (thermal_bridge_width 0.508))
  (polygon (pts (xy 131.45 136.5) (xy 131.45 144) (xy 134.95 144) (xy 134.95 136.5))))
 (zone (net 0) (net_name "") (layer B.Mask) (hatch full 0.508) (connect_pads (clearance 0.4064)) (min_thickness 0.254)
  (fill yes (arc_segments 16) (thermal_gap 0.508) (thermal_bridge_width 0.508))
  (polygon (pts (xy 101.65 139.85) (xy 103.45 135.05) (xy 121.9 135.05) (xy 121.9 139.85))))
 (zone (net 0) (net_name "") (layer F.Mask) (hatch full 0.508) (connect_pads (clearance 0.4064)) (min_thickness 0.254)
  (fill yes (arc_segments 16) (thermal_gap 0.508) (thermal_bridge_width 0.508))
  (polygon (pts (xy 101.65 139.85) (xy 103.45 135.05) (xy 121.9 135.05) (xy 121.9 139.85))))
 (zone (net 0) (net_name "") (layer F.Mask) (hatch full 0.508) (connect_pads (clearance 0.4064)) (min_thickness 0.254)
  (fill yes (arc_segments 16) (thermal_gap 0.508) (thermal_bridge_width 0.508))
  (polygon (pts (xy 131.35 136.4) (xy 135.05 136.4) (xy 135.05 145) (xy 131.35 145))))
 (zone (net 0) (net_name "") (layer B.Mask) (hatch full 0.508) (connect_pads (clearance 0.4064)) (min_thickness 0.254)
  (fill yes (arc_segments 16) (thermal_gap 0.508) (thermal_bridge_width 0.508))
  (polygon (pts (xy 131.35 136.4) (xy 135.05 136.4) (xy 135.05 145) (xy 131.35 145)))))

